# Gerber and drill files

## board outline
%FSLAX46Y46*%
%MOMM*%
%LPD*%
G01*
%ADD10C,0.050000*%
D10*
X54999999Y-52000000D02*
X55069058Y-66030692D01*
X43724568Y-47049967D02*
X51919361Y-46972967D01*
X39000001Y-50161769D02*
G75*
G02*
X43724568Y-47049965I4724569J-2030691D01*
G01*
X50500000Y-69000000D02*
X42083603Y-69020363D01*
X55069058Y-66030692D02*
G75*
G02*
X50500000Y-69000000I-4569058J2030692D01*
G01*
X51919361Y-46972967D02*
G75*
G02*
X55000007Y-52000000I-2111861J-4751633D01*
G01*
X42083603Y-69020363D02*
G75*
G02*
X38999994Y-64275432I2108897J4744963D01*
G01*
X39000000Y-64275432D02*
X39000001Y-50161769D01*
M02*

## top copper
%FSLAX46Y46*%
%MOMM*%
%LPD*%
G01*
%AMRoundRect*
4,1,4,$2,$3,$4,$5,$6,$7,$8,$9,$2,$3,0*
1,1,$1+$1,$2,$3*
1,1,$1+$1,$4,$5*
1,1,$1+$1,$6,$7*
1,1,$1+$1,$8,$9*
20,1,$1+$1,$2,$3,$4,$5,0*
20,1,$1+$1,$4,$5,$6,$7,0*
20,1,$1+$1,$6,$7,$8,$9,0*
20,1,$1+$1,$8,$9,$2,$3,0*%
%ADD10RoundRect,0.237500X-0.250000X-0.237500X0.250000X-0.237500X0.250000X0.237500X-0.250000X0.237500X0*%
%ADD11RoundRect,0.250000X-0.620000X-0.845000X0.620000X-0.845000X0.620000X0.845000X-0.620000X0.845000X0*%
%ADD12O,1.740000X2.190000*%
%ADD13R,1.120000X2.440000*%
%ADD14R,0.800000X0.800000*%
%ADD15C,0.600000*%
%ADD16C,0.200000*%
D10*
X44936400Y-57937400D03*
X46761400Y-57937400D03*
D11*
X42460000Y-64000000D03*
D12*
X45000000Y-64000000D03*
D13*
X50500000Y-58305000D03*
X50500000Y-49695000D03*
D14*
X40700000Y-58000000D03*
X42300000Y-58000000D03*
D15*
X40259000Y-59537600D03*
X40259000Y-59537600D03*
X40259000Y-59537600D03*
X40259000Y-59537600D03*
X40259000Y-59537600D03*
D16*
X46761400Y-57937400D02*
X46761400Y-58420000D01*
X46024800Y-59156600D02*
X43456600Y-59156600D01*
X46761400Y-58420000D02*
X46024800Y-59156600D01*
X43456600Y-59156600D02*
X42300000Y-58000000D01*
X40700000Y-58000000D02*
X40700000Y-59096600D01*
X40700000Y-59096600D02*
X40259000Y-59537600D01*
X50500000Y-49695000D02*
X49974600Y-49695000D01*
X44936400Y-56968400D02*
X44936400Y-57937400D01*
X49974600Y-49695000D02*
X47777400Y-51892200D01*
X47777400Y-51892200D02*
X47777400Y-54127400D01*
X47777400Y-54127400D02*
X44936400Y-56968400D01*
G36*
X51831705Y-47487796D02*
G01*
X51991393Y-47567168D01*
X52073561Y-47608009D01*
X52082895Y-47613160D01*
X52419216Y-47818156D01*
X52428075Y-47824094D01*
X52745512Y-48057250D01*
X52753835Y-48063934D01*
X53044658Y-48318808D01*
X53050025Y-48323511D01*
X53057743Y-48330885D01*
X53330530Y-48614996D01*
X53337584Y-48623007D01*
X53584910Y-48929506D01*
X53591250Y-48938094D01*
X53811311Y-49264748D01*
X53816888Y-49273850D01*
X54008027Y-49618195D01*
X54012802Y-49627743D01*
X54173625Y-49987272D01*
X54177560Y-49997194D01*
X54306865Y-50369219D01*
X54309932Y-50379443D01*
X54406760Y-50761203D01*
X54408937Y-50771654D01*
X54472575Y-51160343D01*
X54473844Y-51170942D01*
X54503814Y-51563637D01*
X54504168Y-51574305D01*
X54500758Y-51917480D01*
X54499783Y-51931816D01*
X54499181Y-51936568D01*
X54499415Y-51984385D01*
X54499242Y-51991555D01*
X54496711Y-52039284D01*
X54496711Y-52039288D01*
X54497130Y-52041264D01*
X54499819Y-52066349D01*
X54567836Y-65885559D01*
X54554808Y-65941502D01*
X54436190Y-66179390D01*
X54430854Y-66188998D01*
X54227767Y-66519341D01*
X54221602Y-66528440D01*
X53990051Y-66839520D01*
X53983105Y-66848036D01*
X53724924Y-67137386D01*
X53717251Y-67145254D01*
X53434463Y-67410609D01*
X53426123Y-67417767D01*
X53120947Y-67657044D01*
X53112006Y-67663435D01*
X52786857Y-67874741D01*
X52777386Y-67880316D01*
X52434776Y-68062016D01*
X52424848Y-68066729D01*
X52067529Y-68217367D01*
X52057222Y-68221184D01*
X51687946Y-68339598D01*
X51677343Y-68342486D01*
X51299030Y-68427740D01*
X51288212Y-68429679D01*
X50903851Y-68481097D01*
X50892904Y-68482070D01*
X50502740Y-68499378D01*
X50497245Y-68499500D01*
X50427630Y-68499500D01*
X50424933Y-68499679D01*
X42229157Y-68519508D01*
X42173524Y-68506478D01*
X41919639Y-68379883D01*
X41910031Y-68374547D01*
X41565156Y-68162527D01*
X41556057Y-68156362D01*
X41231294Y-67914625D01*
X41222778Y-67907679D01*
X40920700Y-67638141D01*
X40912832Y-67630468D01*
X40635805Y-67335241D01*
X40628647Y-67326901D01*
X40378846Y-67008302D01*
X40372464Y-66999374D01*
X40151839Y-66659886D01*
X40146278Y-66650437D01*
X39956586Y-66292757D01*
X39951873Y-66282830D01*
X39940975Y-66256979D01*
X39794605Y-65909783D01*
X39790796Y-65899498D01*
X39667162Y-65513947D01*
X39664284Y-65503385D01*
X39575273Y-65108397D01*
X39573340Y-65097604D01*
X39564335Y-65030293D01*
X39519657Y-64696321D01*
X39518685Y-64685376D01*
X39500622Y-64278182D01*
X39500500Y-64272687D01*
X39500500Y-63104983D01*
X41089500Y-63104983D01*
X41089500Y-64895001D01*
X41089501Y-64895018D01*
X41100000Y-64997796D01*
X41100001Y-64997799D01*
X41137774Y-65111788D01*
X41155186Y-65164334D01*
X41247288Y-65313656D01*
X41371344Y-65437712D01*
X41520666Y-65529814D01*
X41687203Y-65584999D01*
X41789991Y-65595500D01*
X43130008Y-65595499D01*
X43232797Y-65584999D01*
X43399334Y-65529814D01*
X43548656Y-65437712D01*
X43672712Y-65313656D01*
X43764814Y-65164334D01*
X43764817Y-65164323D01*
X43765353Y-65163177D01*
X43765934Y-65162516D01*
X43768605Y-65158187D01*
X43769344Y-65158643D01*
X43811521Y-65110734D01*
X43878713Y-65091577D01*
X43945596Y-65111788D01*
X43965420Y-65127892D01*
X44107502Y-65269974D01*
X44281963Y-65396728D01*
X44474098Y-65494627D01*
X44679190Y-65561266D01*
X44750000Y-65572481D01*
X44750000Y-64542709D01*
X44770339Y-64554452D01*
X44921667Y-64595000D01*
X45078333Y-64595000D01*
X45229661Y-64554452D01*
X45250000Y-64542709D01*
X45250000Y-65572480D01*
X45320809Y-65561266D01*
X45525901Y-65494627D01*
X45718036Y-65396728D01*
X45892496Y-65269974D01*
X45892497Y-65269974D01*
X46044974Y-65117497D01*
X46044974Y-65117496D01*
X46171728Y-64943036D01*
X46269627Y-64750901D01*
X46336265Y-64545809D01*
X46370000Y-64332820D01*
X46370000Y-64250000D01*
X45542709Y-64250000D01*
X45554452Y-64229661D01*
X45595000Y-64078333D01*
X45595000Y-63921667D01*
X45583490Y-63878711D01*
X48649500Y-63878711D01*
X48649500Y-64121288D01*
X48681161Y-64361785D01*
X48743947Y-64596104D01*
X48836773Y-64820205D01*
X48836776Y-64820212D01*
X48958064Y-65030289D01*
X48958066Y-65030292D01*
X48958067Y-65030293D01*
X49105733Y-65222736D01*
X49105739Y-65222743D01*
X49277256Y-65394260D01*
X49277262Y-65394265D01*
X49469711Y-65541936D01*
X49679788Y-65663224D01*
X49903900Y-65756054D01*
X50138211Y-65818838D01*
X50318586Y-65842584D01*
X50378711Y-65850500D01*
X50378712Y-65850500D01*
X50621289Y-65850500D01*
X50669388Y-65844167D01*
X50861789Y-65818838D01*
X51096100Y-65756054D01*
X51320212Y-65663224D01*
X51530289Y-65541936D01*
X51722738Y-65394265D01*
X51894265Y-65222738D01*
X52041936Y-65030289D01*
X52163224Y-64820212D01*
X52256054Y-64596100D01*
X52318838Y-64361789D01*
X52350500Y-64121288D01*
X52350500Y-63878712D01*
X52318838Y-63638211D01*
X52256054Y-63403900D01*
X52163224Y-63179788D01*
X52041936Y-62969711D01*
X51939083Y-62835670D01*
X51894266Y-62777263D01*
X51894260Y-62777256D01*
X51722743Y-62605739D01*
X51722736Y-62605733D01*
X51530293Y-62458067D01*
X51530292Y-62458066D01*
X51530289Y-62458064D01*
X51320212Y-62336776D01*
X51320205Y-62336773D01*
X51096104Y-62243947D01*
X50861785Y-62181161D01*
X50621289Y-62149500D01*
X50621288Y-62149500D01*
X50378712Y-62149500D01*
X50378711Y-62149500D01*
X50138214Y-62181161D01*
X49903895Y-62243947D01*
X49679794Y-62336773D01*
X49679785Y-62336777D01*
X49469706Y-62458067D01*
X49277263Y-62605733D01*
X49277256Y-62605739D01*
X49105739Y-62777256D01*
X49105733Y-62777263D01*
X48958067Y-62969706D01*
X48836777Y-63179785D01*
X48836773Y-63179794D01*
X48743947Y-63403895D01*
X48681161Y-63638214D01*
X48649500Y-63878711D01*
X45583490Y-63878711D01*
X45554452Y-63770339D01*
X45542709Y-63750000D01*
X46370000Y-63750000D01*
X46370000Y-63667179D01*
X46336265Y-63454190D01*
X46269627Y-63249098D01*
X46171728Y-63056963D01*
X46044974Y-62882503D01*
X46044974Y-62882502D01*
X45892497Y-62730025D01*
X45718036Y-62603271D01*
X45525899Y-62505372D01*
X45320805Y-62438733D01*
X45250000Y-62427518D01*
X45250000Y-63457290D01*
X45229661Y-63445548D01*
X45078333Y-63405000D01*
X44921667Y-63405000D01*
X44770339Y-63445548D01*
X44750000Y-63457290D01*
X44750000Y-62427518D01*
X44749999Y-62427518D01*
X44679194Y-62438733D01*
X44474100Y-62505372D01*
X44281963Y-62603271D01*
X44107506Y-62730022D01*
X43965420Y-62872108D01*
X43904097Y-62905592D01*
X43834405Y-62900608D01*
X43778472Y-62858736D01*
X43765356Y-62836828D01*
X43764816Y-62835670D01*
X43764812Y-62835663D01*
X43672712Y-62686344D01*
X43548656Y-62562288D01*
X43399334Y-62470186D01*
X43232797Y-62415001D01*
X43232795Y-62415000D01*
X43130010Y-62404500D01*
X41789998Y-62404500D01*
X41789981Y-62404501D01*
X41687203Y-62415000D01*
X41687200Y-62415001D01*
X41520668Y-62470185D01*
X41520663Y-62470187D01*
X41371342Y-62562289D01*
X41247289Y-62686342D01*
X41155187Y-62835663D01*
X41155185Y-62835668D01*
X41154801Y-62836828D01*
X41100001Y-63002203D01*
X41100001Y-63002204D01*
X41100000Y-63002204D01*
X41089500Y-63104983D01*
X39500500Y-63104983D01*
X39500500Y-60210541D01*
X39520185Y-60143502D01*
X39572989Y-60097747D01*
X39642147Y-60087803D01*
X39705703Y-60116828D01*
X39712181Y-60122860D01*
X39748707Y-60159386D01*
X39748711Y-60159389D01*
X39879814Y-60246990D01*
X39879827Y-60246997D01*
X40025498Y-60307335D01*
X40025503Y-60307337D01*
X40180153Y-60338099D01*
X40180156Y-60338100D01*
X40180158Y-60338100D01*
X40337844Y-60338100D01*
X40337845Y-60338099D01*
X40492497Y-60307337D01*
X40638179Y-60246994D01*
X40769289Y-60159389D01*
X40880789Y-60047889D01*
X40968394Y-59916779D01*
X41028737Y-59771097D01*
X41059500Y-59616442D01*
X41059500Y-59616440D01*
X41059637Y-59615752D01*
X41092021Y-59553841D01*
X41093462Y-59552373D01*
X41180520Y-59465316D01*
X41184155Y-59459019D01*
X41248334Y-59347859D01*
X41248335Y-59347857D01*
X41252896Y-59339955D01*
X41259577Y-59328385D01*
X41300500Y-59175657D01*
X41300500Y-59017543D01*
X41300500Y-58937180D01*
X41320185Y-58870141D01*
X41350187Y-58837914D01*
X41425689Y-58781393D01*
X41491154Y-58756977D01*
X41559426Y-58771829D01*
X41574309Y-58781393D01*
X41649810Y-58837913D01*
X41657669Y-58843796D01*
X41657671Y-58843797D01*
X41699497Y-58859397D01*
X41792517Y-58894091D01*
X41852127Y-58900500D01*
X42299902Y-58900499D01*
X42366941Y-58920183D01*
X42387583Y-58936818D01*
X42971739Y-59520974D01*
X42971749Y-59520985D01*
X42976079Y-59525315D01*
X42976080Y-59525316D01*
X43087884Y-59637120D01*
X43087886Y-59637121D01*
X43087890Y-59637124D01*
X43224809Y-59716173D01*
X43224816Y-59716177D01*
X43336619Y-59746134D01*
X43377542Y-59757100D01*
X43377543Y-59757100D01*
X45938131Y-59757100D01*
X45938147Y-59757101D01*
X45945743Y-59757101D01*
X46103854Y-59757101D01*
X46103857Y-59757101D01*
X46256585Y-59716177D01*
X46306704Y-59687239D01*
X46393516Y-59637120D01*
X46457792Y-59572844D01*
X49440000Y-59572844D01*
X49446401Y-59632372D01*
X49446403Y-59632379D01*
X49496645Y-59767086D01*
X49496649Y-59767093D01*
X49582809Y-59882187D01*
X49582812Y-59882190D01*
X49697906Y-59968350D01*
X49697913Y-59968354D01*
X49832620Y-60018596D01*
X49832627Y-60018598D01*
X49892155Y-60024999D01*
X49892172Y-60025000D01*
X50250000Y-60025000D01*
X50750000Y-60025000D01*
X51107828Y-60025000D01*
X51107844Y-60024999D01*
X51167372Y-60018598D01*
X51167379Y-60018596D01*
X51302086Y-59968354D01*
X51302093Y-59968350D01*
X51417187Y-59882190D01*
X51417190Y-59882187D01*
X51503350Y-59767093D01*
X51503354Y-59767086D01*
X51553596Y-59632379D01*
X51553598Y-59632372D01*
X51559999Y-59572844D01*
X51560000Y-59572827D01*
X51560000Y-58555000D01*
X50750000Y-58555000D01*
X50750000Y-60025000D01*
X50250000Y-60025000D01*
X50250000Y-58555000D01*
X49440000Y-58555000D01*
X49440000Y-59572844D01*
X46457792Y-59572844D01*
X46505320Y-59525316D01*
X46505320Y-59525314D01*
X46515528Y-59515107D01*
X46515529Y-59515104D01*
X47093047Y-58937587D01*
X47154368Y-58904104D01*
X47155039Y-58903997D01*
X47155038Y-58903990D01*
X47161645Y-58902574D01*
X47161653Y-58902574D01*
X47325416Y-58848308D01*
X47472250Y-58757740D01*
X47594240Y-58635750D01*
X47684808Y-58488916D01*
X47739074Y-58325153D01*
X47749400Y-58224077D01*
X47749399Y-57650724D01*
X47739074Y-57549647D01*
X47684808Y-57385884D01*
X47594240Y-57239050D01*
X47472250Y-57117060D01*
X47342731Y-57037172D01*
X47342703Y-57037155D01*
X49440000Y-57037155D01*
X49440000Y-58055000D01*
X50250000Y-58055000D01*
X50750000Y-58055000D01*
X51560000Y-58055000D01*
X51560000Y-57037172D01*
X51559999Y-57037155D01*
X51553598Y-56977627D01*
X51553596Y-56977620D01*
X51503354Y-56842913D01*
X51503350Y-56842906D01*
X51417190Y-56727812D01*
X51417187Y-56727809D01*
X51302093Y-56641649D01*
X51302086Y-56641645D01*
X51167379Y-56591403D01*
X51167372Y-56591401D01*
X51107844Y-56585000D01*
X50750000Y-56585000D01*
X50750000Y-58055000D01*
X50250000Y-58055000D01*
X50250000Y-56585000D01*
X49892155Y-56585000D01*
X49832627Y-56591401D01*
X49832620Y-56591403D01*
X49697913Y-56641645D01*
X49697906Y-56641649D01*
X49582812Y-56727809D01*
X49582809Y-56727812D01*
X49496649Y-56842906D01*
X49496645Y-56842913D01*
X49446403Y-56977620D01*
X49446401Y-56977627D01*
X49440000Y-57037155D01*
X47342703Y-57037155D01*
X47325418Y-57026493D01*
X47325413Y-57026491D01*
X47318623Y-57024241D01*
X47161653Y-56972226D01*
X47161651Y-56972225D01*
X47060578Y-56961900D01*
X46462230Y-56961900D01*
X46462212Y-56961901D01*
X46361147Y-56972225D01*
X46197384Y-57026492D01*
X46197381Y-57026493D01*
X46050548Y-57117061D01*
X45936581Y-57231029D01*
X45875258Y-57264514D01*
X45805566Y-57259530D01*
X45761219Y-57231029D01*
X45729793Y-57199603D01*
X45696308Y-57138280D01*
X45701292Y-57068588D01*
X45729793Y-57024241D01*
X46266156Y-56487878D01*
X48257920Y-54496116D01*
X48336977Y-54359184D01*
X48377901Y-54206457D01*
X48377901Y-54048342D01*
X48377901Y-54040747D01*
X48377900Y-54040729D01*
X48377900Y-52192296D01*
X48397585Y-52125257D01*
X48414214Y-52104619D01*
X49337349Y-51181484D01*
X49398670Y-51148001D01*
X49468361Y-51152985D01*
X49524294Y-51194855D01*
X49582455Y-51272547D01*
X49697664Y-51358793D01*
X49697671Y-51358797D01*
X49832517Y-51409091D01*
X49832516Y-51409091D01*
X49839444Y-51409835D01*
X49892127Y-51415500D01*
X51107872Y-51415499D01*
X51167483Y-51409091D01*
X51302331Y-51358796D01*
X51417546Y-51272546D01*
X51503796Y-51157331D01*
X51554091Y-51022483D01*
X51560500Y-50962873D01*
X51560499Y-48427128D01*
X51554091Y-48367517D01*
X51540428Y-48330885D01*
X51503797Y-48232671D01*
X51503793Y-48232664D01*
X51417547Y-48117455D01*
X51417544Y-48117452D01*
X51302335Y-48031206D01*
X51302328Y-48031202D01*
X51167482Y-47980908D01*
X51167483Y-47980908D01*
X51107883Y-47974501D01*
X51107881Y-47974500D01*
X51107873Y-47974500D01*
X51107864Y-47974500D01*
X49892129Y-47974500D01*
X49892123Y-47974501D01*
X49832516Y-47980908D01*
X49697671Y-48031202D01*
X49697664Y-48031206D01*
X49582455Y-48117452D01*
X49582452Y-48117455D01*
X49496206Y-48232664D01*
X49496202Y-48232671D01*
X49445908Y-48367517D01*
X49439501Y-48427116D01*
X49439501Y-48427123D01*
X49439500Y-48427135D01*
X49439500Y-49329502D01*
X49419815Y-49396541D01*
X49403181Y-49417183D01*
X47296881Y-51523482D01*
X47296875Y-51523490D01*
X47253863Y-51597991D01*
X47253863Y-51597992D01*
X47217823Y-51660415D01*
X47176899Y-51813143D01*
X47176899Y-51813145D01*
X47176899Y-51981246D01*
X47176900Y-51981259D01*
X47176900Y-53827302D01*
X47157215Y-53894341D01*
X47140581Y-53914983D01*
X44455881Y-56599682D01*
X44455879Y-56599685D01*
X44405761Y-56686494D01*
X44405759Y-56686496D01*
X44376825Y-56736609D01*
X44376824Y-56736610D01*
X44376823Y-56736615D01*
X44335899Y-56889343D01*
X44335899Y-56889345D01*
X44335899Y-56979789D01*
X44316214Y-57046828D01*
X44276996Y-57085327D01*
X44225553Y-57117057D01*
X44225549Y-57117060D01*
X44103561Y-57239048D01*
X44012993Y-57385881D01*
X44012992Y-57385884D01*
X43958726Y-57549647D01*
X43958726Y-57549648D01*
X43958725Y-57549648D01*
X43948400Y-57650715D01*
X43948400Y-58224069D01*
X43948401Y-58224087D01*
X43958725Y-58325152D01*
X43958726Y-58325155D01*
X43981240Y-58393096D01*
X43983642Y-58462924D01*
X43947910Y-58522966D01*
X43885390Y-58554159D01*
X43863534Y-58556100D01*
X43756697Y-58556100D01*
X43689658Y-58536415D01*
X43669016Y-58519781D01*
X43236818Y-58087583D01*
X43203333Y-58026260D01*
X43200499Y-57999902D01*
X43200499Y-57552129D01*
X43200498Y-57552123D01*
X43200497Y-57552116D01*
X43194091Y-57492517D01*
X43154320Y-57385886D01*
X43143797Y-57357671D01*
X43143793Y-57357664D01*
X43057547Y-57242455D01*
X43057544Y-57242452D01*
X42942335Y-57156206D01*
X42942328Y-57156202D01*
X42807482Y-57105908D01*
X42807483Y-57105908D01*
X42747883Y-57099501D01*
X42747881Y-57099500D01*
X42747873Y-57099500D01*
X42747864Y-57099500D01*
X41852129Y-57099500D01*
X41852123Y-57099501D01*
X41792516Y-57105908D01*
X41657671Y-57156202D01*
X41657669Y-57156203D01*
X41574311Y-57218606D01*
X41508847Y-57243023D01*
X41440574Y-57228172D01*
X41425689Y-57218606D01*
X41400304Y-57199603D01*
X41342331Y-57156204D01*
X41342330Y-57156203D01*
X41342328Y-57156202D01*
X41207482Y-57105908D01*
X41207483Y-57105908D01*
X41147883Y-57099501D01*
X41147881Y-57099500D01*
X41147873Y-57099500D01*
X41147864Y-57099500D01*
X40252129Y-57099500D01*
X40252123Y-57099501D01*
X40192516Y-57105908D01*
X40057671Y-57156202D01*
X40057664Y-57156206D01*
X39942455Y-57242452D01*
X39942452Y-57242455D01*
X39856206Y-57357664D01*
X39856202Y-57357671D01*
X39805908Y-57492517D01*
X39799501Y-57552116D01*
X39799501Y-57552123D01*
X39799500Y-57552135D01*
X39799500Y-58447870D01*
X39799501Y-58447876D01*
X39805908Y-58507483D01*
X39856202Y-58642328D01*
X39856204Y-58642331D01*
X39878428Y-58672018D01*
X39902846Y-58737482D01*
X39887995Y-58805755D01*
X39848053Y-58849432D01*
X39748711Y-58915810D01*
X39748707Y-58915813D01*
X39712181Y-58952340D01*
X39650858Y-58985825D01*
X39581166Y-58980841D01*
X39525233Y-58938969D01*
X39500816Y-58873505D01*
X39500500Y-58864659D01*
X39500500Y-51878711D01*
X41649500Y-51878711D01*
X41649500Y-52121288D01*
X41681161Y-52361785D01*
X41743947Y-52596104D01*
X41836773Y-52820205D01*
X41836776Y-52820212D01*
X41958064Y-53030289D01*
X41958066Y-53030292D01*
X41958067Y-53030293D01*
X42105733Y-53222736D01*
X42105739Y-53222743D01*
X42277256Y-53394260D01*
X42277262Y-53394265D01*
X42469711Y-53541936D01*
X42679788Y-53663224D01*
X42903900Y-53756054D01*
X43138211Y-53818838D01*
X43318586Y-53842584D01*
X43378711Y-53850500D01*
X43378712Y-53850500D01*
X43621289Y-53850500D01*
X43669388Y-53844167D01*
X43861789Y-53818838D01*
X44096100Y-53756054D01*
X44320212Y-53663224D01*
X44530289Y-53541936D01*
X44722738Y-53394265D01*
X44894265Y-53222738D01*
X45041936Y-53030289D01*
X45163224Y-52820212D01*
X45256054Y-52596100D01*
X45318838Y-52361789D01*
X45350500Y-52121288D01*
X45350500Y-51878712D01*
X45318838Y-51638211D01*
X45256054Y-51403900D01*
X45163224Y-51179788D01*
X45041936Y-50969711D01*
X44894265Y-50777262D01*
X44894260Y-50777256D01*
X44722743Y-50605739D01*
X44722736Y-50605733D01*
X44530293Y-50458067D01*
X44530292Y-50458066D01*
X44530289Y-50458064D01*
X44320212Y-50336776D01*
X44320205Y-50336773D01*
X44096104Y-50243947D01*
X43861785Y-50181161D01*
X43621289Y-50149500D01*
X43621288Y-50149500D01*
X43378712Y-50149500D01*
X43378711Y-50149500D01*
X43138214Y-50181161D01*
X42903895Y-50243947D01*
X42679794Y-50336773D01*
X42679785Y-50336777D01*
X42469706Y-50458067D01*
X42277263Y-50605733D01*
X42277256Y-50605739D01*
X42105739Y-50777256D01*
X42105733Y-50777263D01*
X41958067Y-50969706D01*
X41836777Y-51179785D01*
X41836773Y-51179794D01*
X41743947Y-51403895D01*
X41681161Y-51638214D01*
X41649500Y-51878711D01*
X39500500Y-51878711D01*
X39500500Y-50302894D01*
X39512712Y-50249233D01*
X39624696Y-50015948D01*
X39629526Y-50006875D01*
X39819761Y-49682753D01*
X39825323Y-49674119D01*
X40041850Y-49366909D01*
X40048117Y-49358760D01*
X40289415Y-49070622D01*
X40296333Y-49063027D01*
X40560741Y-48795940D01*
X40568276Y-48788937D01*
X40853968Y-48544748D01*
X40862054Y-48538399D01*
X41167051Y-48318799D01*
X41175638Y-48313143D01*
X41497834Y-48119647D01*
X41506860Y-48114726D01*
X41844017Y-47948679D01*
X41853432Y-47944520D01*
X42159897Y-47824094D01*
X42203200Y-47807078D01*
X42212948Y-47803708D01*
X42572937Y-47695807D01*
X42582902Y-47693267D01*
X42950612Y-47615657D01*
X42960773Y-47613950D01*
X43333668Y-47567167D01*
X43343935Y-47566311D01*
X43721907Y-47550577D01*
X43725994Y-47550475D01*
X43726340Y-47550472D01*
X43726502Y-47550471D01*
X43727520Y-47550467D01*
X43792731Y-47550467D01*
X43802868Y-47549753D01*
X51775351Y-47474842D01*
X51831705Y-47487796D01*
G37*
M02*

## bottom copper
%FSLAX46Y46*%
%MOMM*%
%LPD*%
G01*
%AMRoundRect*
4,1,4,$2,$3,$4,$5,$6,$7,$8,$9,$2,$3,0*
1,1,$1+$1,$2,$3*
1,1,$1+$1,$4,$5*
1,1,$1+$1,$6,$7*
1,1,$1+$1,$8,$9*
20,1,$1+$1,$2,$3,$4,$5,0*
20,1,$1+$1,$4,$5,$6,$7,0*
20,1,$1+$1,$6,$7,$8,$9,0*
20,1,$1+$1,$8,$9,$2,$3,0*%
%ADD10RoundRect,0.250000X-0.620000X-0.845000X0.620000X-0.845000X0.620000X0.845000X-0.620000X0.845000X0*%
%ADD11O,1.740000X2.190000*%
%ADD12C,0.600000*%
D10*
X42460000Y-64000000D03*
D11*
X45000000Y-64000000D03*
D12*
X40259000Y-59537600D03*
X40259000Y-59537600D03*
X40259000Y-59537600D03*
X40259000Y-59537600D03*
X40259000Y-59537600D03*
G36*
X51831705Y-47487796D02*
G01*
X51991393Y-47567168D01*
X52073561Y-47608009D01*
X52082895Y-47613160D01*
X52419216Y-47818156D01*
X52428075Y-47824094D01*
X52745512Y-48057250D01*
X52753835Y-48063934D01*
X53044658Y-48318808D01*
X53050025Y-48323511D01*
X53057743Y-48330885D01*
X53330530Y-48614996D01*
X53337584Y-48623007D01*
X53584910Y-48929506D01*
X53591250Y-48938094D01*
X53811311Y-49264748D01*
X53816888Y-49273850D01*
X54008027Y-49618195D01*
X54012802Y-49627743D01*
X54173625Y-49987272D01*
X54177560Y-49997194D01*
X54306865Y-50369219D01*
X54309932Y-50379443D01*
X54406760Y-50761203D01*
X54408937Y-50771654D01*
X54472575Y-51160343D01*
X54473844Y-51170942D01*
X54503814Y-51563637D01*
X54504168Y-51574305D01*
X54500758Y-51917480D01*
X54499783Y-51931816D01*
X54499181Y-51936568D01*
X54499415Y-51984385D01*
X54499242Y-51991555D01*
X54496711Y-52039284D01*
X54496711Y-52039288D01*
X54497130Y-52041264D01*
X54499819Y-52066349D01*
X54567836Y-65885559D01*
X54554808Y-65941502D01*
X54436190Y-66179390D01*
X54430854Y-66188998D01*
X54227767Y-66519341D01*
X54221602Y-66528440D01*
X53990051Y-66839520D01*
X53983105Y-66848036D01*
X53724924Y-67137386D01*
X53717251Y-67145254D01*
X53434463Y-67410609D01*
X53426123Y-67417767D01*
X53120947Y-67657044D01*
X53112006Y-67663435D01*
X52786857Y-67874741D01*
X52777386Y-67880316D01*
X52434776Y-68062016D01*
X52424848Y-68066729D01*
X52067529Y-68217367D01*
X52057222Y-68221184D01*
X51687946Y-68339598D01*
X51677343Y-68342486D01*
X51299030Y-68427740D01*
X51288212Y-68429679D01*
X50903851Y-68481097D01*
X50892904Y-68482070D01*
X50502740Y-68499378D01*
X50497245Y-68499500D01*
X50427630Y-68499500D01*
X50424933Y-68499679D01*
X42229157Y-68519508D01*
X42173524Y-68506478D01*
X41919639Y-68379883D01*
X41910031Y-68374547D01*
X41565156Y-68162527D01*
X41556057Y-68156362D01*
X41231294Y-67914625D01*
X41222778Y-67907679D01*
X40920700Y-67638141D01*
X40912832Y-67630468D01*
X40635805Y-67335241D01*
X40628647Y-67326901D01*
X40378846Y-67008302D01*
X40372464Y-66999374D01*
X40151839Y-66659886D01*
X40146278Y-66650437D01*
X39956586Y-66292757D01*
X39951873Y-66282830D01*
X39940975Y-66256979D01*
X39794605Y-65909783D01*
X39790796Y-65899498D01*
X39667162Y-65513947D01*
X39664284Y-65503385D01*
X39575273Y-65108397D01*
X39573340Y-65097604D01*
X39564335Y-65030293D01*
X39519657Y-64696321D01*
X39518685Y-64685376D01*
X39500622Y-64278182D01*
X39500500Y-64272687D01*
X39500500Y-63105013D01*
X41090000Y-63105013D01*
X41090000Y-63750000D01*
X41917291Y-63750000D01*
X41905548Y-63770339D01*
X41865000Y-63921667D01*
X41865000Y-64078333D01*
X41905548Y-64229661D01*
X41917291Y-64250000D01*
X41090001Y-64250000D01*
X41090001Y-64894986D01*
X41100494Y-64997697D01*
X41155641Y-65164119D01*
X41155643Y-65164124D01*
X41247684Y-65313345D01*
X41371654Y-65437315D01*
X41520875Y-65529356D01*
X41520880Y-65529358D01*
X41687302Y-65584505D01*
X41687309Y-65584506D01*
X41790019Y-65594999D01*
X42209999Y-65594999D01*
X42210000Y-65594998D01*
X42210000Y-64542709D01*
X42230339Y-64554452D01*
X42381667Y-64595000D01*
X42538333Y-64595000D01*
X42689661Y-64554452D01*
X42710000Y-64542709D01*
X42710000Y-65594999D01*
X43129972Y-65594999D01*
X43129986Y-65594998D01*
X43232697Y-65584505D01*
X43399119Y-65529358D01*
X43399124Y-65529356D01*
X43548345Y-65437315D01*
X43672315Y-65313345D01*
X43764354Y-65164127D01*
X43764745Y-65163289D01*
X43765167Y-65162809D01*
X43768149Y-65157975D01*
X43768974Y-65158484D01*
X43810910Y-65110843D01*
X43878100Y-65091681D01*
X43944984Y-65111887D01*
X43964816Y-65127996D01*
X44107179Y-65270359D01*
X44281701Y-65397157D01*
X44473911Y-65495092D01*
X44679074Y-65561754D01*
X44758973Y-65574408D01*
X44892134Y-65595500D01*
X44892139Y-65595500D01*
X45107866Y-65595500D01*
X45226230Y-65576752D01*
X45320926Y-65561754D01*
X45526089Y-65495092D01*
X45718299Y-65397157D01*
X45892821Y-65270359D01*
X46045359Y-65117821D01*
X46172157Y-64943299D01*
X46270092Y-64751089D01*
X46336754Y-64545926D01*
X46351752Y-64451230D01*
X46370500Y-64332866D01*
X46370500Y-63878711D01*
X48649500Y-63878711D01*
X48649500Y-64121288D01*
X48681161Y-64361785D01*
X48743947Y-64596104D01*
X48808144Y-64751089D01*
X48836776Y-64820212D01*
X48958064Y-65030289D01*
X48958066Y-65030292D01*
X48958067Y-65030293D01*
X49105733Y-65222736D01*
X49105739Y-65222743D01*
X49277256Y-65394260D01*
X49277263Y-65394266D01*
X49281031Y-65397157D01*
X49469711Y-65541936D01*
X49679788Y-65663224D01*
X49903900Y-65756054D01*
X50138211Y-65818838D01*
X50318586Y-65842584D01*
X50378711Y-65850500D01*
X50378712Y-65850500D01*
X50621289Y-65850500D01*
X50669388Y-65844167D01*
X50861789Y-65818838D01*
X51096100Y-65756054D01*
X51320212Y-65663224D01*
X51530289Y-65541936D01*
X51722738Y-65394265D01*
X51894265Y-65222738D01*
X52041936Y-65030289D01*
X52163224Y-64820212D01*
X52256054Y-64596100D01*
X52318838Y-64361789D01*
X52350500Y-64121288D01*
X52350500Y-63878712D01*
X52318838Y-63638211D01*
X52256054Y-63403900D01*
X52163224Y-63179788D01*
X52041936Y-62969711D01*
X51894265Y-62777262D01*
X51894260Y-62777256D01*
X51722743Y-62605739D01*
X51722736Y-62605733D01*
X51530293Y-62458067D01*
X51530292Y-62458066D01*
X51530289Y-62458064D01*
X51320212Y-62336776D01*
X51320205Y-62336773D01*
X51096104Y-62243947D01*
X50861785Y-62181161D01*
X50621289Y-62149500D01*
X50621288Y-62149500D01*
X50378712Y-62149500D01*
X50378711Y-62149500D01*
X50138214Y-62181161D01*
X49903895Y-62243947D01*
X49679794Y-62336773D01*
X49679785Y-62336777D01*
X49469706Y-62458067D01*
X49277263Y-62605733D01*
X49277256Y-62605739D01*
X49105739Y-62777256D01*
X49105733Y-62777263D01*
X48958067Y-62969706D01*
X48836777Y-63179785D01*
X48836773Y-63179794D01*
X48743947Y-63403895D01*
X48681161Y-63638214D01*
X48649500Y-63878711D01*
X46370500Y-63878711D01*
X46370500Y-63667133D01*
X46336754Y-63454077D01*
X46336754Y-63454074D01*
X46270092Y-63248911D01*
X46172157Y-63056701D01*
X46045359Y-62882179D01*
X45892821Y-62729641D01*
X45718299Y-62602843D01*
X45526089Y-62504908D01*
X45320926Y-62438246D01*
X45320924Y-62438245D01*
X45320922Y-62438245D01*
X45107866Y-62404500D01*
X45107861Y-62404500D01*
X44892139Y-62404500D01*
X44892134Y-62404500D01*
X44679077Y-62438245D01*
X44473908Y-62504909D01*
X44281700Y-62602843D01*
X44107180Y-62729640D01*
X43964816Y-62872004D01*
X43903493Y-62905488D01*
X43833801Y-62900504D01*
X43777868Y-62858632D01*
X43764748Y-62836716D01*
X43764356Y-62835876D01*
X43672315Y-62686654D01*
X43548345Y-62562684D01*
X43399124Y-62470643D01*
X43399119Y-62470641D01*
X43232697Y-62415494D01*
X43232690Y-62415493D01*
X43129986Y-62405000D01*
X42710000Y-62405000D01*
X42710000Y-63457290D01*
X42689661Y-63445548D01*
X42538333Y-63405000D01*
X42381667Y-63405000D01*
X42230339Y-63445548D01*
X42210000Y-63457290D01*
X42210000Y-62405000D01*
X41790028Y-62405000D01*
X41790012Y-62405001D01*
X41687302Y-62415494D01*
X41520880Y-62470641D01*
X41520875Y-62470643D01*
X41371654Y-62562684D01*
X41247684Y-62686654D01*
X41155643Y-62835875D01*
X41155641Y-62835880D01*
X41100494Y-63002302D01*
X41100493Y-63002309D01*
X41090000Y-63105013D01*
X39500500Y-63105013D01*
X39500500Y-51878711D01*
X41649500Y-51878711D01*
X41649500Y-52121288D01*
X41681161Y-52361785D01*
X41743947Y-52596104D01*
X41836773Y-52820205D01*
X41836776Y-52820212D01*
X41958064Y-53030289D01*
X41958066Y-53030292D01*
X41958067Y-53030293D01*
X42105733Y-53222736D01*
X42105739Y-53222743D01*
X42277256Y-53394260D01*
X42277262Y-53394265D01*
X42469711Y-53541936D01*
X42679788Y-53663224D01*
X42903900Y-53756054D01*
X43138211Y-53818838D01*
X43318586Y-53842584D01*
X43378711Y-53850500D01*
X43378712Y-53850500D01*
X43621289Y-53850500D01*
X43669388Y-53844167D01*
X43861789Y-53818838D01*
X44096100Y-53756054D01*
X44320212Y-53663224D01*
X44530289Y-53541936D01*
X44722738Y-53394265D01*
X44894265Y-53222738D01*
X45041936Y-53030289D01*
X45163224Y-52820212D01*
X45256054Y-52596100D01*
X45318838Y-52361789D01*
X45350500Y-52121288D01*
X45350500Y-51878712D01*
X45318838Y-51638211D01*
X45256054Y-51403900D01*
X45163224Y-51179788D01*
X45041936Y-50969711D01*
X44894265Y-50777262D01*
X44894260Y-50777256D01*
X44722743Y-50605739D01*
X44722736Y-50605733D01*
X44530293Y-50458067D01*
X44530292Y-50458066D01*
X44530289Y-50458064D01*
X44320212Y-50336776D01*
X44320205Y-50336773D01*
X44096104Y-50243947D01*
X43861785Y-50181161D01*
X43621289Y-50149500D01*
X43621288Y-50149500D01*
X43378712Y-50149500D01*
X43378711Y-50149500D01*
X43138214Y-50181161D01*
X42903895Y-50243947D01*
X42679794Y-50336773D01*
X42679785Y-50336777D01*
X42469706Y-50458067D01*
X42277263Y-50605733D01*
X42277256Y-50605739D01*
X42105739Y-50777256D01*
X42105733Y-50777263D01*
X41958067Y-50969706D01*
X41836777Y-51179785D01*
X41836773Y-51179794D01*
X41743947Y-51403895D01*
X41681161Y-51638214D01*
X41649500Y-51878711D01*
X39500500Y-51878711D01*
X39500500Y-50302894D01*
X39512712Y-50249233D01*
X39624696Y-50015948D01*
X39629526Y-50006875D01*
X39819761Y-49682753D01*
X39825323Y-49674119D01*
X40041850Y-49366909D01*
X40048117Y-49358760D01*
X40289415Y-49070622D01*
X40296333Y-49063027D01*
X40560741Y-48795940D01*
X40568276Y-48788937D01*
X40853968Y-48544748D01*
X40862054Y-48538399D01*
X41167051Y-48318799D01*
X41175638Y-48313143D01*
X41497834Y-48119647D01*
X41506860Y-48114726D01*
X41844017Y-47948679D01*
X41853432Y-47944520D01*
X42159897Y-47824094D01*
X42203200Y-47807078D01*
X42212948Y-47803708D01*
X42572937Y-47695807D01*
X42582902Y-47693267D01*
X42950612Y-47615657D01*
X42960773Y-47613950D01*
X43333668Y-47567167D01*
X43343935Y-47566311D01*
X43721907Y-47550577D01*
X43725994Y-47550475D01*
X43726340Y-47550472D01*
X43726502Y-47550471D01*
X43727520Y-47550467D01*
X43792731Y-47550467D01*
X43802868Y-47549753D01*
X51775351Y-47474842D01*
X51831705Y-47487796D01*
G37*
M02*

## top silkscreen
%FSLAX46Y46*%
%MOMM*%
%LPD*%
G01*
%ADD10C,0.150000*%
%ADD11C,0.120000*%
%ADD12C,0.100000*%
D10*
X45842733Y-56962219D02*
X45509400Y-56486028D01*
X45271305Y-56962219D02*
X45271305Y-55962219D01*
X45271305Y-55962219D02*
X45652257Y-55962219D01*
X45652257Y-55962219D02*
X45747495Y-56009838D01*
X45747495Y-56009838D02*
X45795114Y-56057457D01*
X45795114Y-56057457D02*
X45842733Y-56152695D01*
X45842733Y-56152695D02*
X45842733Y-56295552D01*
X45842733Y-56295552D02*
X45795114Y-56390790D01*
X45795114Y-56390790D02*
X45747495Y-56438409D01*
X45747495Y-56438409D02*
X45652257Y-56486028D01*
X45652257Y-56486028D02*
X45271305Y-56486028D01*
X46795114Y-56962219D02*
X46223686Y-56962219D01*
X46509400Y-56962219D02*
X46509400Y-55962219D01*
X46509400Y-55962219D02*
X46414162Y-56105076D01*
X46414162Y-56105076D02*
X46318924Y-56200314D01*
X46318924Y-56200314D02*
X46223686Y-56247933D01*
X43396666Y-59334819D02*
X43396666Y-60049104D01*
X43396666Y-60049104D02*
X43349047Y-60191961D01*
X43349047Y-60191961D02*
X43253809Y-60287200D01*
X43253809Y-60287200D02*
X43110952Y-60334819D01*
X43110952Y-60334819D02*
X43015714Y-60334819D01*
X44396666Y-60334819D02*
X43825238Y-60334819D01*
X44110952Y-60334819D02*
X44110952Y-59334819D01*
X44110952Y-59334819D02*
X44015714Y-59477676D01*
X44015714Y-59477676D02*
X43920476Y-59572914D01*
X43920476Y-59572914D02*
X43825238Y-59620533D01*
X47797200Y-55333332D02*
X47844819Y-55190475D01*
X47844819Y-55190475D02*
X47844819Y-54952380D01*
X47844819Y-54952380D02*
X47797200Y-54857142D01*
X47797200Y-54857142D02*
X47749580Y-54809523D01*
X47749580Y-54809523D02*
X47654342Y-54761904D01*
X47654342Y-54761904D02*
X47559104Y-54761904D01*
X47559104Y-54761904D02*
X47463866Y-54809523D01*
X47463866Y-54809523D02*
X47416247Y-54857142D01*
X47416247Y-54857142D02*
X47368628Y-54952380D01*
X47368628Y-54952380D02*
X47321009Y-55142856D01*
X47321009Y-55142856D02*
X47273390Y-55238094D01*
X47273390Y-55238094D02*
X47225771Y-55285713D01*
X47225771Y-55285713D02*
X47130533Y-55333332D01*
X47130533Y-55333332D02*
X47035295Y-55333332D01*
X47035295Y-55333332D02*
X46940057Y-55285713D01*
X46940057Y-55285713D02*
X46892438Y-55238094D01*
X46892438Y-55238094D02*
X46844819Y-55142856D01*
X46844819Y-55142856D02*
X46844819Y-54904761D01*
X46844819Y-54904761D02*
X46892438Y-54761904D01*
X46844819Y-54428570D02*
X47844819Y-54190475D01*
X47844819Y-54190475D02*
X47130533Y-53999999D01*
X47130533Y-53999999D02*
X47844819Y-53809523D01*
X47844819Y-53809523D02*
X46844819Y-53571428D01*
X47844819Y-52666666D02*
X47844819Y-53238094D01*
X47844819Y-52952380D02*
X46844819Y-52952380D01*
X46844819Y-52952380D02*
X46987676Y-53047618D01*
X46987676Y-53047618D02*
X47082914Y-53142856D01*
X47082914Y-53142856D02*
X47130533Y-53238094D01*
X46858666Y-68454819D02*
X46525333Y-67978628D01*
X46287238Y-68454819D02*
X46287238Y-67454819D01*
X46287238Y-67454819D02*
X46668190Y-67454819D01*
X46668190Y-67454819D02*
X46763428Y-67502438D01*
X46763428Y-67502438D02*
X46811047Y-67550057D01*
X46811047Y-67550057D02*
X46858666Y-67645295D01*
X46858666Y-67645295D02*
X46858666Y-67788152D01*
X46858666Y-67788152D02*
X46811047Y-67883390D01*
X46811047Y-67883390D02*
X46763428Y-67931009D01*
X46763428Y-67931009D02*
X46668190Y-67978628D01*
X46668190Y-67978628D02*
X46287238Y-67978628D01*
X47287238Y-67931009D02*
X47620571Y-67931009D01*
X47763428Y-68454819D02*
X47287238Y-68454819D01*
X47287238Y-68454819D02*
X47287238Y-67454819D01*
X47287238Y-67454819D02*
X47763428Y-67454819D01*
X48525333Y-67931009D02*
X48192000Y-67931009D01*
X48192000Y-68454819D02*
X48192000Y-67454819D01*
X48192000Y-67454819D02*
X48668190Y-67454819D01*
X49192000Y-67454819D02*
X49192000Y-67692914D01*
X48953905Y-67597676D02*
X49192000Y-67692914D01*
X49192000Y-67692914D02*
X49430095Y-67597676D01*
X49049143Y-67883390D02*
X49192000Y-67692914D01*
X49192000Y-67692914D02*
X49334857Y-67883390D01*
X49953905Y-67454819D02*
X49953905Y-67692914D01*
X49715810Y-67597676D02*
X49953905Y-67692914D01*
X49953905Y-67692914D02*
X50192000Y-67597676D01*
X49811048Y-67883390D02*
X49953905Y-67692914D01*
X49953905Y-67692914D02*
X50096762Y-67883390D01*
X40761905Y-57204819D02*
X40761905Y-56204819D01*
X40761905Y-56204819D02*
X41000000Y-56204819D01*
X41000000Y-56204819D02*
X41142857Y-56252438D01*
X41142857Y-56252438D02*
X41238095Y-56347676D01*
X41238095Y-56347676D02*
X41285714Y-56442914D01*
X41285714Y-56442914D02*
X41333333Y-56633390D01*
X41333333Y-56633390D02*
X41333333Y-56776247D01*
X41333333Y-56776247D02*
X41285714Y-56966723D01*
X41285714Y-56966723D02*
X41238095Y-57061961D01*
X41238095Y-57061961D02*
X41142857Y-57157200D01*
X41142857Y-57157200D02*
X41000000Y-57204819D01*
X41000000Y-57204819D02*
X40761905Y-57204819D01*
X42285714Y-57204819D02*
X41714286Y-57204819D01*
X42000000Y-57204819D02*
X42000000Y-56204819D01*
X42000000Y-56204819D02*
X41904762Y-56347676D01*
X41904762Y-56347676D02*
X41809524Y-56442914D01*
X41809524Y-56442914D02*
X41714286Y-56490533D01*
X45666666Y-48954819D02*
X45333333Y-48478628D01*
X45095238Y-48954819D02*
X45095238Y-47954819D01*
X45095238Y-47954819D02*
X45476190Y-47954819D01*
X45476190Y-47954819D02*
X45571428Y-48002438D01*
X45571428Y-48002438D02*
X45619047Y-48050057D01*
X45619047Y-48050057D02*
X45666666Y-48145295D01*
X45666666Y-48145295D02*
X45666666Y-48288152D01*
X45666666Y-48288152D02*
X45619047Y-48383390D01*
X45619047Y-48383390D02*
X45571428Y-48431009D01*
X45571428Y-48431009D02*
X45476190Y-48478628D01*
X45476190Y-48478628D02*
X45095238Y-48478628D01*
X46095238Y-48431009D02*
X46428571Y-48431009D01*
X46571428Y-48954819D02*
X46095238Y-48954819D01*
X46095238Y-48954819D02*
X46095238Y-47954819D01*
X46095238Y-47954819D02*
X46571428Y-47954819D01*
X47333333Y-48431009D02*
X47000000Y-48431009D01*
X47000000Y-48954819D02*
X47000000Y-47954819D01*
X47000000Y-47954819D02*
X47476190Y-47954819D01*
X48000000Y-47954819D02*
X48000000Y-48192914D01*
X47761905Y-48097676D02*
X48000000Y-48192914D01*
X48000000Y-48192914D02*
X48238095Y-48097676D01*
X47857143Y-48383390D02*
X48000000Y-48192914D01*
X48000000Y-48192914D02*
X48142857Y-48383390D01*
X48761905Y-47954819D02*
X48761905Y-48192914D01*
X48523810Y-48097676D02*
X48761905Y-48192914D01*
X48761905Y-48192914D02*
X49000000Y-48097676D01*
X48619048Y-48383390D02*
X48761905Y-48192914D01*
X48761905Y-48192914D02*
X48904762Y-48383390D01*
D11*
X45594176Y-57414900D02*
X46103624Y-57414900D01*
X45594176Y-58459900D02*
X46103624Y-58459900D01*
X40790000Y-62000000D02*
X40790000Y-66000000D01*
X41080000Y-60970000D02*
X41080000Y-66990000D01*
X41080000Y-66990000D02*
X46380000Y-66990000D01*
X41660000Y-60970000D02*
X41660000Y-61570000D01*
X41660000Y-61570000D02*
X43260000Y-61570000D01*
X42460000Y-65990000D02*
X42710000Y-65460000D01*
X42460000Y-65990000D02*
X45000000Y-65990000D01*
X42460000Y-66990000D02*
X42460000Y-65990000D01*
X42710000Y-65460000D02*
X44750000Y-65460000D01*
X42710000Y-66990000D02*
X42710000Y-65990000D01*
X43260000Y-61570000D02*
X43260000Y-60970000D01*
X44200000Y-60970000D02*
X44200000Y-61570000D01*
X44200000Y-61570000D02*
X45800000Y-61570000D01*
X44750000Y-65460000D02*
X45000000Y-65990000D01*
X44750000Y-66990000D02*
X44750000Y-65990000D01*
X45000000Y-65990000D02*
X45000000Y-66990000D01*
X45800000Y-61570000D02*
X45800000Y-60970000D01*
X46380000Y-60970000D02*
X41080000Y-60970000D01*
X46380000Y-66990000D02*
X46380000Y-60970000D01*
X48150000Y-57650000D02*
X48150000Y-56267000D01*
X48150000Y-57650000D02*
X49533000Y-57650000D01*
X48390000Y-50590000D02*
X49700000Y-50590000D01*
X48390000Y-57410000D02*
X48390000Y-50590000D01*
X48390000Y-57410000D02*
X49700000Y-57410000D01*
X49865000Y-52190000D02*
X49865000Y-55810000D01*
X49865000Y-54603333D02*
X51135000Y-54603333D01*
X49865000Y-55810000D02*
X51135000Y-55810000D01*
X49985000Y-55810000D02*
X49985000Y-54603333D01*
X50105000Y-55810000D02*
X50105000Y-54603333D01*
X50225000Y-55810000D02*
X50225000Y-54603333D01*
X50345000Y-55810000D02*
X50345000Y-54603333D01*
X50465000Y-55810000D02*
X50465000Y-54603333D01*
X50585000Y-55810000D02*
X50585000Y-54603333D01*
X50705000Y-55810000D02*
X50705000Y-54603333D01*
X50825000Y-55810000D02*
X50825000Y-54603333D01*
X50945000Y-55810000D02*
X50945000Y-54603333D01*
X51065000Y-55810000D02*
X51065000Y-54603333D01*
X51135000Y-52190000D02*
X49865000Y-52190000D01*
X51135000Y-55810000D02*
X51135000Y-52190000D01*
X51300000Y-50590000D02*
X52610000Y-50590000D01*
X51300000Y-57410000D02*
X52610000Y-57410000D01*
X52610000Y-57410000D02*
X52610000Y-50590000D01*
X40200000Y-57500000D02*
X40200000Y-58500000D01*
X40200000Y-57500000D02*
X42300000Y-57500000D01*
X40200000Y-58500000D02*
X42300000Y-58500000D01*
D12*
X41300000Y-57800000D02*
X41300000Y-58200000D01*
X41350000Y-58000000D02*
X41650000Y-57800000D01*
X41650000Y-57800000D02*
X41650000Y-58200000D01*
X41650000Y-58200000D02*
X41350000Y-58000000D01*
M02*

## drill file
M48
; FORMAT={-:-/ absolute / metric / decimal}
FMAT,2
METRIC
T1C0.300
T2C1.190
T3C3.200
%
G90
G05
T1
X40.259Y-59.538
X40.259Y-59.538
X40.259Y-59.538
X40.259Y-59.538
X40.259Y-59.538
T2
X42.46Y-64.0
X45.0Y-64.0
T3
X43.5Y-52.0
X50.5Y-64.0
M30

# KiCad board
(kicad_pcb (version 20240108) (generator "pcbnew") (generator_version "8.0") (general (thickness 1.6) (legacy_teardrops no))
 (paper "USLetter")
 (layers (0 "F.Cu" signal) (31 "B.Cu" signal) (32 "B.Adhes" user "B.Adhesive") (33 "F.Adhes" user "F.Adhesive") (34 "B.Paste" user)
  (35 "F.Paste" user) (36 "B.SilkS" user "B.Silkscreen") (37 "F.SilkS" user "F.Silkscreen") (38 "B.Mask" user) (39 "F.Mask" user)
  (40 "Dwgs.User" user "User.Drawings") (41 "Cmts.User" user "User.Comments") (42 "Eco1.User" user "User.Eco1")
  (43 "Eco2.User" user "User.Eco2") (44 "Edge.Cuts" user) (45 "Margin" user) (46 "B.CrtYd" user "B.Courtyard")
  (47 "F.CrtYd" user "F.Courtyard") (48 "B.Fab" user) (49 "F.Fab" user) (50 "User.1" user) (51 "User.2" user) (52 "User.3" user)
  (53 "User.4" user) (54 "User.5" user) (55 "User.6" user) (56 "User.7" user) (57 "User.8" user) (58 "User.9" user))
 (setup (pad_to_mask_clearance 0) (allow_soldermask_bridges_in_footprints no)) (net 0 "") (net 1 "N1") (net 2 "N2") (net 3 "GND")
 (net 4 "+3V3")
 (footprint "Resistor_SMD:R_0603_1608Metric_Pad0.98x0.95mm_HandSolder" (layer "F.Cu") (at 45.8489 57.9374)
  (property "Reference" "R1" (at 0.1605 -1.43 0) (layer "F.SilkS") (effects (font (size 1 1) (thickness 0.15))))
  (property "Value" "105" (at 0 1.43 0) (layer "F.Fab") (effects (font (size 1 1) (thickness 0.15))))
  (fp_line (start -0.254724 -0.5225) (end 0.254724 -0.5225) (stroke (width 0.12) (type solid)) (layer "F.SilkS"))
  (fp_line (start -0.254724 0.5225) (end 0.254724 0.5225) (stroke (width 0.12) (type solid)) (layer "F.SilkS"))
  (pad "1" smd roundrect (at -0.9125 0) (size 0.975 0.95) (layers "F.Cu" "F.Paste" "F.Mask") (roundrect_rratio 0.25) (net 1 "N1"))
  (pad "2" smd roundrect (at 0.9125 0) (size 0.975 0.95) (layers "F.Cu" "F.Paste" "F.Mask") (roundrect_rratio 0.25) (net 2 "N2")))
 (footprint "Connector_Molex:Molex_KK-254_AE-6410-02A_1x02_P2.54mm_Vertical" (layer "F.Cu") (at 42.46 64)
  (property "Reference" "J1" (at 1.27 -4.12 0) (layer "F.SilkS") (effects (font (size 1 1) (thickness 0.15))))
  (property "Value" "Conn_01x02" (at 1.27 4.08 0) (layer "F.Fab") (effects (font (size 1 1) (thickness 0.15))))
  (fp_line (start -1.67 -2) (end -1.67 2) (stroke (width 0.12) (type solid)) (layer "F.SilkS"))
  (fp_line (start -1.38 -3.03) (end -1.38 2.99) (stroke (width 0.12) (type solid)) (layer "F.SilkS"))
  (fp_line (start -1.38 2.99) (end 3.92 2.99) (stroke (width 0.12) (type solid)) (layer "F.SilkS"))
  (fp_line (start -0.8 -3.03) (end -0.8 -2.43) (stroke (width 0.12) (type solid)) (layer "F.SilkS"))
  (fp_line (start -0.8 -2.43) (end 0.8 -2.43) (stroke (width 0.12) (type solid)) (layer "F.SilkS"))
  (fp_line (start 0 1.99) (end 0.25 1.46) (stroke (width 0.12) (type solid)) (layer "F.SilkS"))
  (fp_line (start 0 1.99) (end 2.54 1.99) (stroke (width 0.12) (type solid)) (layer "F.SilkS"))
  (fp_line (start 0 2.99) (end 0 1.99) (stroke (width 0.12) (type solid)) (layer "F.SilkS"))
  (fp_line (start 0.25 1.46) (end 2.29 1.46) (stroke (width 0.12) (type solid)) (layer "F.SilkS"))
  (fp_line (start 0.25 2.99) (end 0.25 1.99) (stroke (width 0.12) (type solid)) (layer "F.SilkS"))
  (fp_line (start 0.8 -2.43) (end 0.8 -3.03) (stroke (width 0.12) (type solid)) (layer "F.SilkS"))
  (fp_line (start 1.74 -3.03) (end 1.74 -2.43) (stroke (width 0.12) (type solid)) (layer "F.SilkS"))
  (fp_line (start 1.74 -2.43) (end 3.34 -2.43) (stroke (width 0.12) (type solid)) (layer "F.SilkS"))
  (fp_line (start 2.29 1.46) (end 2.54 1.99) (stroke (width 0.12) (type solid)) (layer "F.SilkS"))
  (fp_line (start 2.29 2.99) (end 2.29 1.99) (stroke (width 0.12) (type solid)) (layer "F.SilkS"))
  (fp_line (start 2.54 1.99) (end 2.54 2.99) (stroke (width 0.12) (type solid)) (layer "F.SilkS"))
  (fp_line (start 3.34 -2.43) (end 3.34 -3.03) (stroke (width 0.12) (type solid)) (layer "F.SilkS"))
  (fp_line (start 3.92 -3.03) (end -1.38 -3.03) (stroke (width 0.12) (type solid)) (layer "F.SilkS"))
  (fp_line (start 3.92 2.99) (end 3.92 -3.03) (stroke (width 0.12) (type solid)) (layer "F.SilkS"))
  (pad "1" thru_hole roundrect (at 0 0) (size 1.74 2.19) (drill 1.19) (layers "*.Cu" "*.Mask") (remove_unused_layers no)
   (roundrect_rratio 0.143678) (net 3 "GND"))
  (pad "2" thru_hole oval (at 2.54 0) (size 1.74 2.19) (drill 1.19) (layers "*.Cu" "*.Mask") (remove_unused_layers no) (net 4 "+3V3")))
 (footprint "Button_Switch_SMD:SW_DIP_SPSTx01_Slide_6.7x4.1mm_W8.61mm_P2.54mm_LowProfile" (layer "F.Cu") (at 50.5 54 90)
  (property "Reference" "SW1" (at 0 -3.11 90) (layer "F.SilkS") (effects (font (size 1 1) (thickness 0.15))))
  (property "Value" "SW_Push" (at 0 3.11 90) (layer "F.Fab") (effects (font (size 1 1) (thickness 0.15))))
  (fp_line (start -3.65 -2.35) (end -2.267 -2.35) (stroke (width 0.12) (type solid)) (layer "F.SilkS"))
  (fp_line (start -3.65 -2.35) (end -3.65 -0.967) (stroke (width 0.12) (type solid)) (layer "F.SilkS"))
  (fp_line (start 3.41 -2.11) (end 3.41 -0.8) (stroke (width 0.12) (type solid)) (layer "F.SilkS"))
  (fp_line (start -3.41 -2.11) (end 3.41 -2.11) (stroke (width 0.12) (type solid)) (layer "F.SilkS"))
  (fp_line (start -3.41 -2.11) (end -3.41 -0.8) (stroke (width 0.12) (type solid)) (layer "F.SilkS"))
  (fp_line (start 1.81 -0.635) (end -1.81 -0.635) (stroke (width 0.12) (type solid)) (layer "F.SilkS"))
  (fp_line (start -0.603333 -0.635) (end -0.603333 0.635) (stroke (width 0.12) (type solid)) (layer "F.SilkS"))
  (fp_line (start -1.81 -0.635) (end -1.81 0.635) (stroke (width 0.12) (type solid)) (layer "F.SilkS"))
  (fp_line (start -1.81 -0.515) (end -0.603333 -0.515) (stroke (width 0.12) (type solid)) (layer "F.SilkS"))
  (fp_line (start -1.81 -0.395) (end -0.603333 -0.395) (stroke (width 0.12) (type solid)) (layer "F.SilkS"))
  (fp_line (start -1.81 -0.275) (end -0.603333 -0.275) (stroke (width 0.12) (type solid)) (layer "F.SilkS"))
  (fp_line (start -1.81 -0.155) (end -0.603333 -0.155) (stroke (width 0.12) (type solid)) (layer "F.SilkS"))
  (fp_line (start -1.81 -0.035) (end -0.603333 -0.035) (stroke (width 0.12) (type solid)) (layer "F.SilkS"))
  (fp_line (start -1.81 0.085) (end -0.603333 0.085) (stroke (width 0.12) (type solid)) (layer "F.SilkS"))
  (fp_line (start -1.81 0.205) (end -0.603333 0.205) (stroke (width 0.12) (type solid)) (layer "F.SilkS"))
  (fp_line (start -1.81 0.325) (end -0.603333 0.325) (stroke (width 0.12) (type solid)) (layer "F.SilkS"))
  (fp_line (start -1.81 0.445) (end -0.603333 0.445) (stroke (width 0.12) (type solid)) (layer "F.SilkS"))
  (fp_line (start -1.81 0.565) (end -0.603333 0.565) (stroke (width 0.12) (type solid)) (layer "F.SilkS"))
  (fp_line (start 1.81 0.635) (end 1.81 -0.635) (stroke (width 0.12) (type solid)) (layer "F.SilkS"))
  (fp_line (start -1.81 0.635) (end 1.81 0.635) (stroke (width 0.12) (type solid)) (layer "F.SilkS"))
  (fp_line (start 3.41 0.8) (end 3.41 2.11) (stroke (width 0.12) (type solid)) (layer "F.SilkS"))
  (fp_line (start -3.41 0.8) (end -3.41 2.11) (stroke (width 0.12) (type solid)) (layer "F.SilkS"))
  (fp_line (start -3.41 2.11) (end 3.41 2.11) (stroke (width 0.12) (type solid)) (layer "F.SilkS"))
  (pad "1" smd rect (at -4.305 0 90) (size 2.44 1.12) (layers "F.Cu" "F.Paste" "F.Mask") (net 4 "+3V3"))
  (pad "2" smd rect (at 4.305 0 90) (size 2.44 1.12) (layers "F.Cu" "F.Paste" "F.Mask") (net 1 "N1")))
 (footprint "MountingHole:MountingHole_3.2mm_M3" (layer "F.Cu") (at 50.5 64)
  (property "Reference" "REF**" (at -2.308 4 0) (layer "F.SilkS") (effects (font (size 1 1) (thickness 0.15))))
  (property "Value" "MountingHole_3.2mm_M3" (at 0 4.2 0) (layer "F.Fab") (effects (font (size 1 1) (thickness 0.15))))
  (pad "" np_thru_hole circle (at 0 0) (size 3.2 3.2) (drill 3.2) (layers "*.Cu" "*.Mask")))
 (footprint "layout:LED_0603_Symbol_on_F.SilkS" (layer "F.Cu") (at 41.5 58)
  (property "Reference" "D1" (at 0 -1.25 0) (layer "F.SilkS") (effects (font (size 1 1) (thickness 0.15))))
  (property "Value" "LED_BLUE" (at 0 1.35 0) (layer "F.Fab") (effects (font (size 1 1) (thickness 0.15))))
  (fp_line (start -1.3 -0.5) (end -1.3 0.5) (stroke (width 0.12) (type solid)) (layer "F.SilkS"))
  (fp_line (start -1.3 -0.5) (end 0.8 -0.5) (stroke (width 0.12) (type solid)) (layer "F.SilkS"))
  (fp_line (start -1.3 0.5) (end 0.8 0.5) (stroke (width 0.12) (type solid)) (layer "F.SilkS"))
  (fp_line (start -0.2 -0.2) (end -0.2 0.2) (stroke (width 0.1) (type solid)) (layer "F.SilkS"))
  (fp_line (start -0.15 0) (end 0.15 -0.2) (stroke (width 0.1) (type solid)) (layer "F.SilkS"))
  (fp_line (start 0.15 -0.2) (end 0.15 0.2) (stroke (width 0.1) (type solid)) (layer "F.SilkS"))
  (fp_line (start 0.15 0.2) (end -0.15 0) (stroke (width 0.1) (type solid)) (layer "F.SilkS"))
  (pad "1" smd rect (at -0.8 0 180) (size 0.8 0.8) (layers "F.Cu" "F.Paste" "F.Mask") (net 3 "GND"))
  (pad "2" smd rect (at 0.8 0 180) (size 0.8 0.8) (layers "F.Cu" "F.Paste" "F.Mask") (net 2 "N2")))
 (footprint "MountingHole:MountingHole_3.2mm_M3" (layer "F.Cu") (at 43.5 52)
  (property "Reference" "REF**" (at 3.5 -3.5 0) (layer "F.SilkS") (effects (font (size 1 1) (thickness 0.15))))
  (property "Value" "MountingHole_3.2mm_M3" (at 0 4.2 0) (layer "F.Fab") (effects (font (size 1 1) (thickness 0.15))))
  (pad "" np_thru_hole circle (at 0 0) (size 3.2 3.2) (drill 3.2) (layers "*.Cu" "*.Mask")))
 (gr_line (start 54.999999 52) (end 55.069058 66.030692) (stroke (width 0.05) (type default)) (layer "Edge.Cuts"))
 (gr_line (start 43.724568 47.049967) (end 51.919361 46.972967) (stroke (width 0.05) (type default)) (layer "Edge.Cuts"))
 (gr_arc (start 39.000001 50.161769) (mid 40.895927 47.897809) (end 43.724568 47.049967) (stroke (width 0.05) (type default))
  (layer "Edge.Cuts"))
 (gr_line (start 50.5 69) (end 42.083603 69.020363) (stroke (width 0.05) (type default)) (layer "Edge.Cuts"))
 (gr_arc (start 55.069058 66.030692) (mid 53.224568 68.192461) (end 50.5 69) (stroke (width 0.05) (type default)) (layer "Edge.Cuts"))
 (gr_arc (start 51.919361 46.972967) (mid 54.241036 49.007657) (end 54.999999 52) (stroke (width 0.05) (type default)) (layer "Edge.Cuts"))
 (gr_arc (start 42.083603 69.020363) (mid 39.838623 67.104874) (end 39 64.275432) (stroke (width 0.05) (type default)) (layer "Edge.Cuts"))
 (gr_line (start 39 64.275432) (end 39.000001 50.161769) (stroke (width 0.05) (type default)) (layer "Edge.Cuts"))
 (segment (start 46.7614 57.9374) (end 46.7614 58.42) (width 0.2) (layer "F.Cu") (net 2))
 (segment (start 46.0248 59.1566) (end 43.4566 59.1566) (width 0.2) (layer "F.Cu") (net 2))
 (segment (start 46.7614 58.42) (end 46.0248 59.1566) (width 0.2) (layer "F.Cu") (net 2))
 (segment (start 43.4566 59.1566) (end 42.3 58) (width 0.2) (layer "F.Cu") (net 2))
 (segment (start 40.7 58) (end 40.7 59.0966) (width 0.2) (layer "F.Cu") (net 3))
 (segment (start 40.7 59.0966) (end 40.259 59.5376) (width 0.2) (layer "F.Cu") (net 3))
 (via (at 40.259 59.5376) (size 0.6) (drill 0.3) (layers "F.Cu" "B.Cu") (free yes) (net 3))
 (via (at 40.259 59.5376) (size 0.6) (drill 0.3) (layers "F.Cu" "B.Cu") (free yes) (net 3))
 (via (at 40.259 59.5376) (size 0.6) (drill 0.3) (layers "F.Cu" "B.Cu") (free yes) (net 3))
 (via (at 40.259 59.5376) (size 0.6) (drill 0.3) (layers "F.Cu" "B.Cu") (free yes) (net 3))
 (via (at 40.259 59.5376) (size 0.6) (drill 0.3) (layers "F.Cu" "B.Cu") (free yes) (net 3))
 (segment (start 50.5 49.695) (end 49.9746 49.695) (width 0.2) (layer "F.Cu") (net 1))
 (segment (start 44.9364 56.9684) (end 44.9364 57.9374) (width 0.2) (layer "F.Cu") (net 1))
 (segment (start 49.9746 49.695) (end 47.7774 51.8922) (width 0.2) (layer "F.Cu") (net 1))
 (segment (start 47.7774 51.8922) (end 47.7774 54.1274) (width 0.2) (layer "F.Cu") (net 1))
 (segment (start 47.7774 54.1274) (end 44.9364 56.9684) (width 0.2) (layer "F.Cu") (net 1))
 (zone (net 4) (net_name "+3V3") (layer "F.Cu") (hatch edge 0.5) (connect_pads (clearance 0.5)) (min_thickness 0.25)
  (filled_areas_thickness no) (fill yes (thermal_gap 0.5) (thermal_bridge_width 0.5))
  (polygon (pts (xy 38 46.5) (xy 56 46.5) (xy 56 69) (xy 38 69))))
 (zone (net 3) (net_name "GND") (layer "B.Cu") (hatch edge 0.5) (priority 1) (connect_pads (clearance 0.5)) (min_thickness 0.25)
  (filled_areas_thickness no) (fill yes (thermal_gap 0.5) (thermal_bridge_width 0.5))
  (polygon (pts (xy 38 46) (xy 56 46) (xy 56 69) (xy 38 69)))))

